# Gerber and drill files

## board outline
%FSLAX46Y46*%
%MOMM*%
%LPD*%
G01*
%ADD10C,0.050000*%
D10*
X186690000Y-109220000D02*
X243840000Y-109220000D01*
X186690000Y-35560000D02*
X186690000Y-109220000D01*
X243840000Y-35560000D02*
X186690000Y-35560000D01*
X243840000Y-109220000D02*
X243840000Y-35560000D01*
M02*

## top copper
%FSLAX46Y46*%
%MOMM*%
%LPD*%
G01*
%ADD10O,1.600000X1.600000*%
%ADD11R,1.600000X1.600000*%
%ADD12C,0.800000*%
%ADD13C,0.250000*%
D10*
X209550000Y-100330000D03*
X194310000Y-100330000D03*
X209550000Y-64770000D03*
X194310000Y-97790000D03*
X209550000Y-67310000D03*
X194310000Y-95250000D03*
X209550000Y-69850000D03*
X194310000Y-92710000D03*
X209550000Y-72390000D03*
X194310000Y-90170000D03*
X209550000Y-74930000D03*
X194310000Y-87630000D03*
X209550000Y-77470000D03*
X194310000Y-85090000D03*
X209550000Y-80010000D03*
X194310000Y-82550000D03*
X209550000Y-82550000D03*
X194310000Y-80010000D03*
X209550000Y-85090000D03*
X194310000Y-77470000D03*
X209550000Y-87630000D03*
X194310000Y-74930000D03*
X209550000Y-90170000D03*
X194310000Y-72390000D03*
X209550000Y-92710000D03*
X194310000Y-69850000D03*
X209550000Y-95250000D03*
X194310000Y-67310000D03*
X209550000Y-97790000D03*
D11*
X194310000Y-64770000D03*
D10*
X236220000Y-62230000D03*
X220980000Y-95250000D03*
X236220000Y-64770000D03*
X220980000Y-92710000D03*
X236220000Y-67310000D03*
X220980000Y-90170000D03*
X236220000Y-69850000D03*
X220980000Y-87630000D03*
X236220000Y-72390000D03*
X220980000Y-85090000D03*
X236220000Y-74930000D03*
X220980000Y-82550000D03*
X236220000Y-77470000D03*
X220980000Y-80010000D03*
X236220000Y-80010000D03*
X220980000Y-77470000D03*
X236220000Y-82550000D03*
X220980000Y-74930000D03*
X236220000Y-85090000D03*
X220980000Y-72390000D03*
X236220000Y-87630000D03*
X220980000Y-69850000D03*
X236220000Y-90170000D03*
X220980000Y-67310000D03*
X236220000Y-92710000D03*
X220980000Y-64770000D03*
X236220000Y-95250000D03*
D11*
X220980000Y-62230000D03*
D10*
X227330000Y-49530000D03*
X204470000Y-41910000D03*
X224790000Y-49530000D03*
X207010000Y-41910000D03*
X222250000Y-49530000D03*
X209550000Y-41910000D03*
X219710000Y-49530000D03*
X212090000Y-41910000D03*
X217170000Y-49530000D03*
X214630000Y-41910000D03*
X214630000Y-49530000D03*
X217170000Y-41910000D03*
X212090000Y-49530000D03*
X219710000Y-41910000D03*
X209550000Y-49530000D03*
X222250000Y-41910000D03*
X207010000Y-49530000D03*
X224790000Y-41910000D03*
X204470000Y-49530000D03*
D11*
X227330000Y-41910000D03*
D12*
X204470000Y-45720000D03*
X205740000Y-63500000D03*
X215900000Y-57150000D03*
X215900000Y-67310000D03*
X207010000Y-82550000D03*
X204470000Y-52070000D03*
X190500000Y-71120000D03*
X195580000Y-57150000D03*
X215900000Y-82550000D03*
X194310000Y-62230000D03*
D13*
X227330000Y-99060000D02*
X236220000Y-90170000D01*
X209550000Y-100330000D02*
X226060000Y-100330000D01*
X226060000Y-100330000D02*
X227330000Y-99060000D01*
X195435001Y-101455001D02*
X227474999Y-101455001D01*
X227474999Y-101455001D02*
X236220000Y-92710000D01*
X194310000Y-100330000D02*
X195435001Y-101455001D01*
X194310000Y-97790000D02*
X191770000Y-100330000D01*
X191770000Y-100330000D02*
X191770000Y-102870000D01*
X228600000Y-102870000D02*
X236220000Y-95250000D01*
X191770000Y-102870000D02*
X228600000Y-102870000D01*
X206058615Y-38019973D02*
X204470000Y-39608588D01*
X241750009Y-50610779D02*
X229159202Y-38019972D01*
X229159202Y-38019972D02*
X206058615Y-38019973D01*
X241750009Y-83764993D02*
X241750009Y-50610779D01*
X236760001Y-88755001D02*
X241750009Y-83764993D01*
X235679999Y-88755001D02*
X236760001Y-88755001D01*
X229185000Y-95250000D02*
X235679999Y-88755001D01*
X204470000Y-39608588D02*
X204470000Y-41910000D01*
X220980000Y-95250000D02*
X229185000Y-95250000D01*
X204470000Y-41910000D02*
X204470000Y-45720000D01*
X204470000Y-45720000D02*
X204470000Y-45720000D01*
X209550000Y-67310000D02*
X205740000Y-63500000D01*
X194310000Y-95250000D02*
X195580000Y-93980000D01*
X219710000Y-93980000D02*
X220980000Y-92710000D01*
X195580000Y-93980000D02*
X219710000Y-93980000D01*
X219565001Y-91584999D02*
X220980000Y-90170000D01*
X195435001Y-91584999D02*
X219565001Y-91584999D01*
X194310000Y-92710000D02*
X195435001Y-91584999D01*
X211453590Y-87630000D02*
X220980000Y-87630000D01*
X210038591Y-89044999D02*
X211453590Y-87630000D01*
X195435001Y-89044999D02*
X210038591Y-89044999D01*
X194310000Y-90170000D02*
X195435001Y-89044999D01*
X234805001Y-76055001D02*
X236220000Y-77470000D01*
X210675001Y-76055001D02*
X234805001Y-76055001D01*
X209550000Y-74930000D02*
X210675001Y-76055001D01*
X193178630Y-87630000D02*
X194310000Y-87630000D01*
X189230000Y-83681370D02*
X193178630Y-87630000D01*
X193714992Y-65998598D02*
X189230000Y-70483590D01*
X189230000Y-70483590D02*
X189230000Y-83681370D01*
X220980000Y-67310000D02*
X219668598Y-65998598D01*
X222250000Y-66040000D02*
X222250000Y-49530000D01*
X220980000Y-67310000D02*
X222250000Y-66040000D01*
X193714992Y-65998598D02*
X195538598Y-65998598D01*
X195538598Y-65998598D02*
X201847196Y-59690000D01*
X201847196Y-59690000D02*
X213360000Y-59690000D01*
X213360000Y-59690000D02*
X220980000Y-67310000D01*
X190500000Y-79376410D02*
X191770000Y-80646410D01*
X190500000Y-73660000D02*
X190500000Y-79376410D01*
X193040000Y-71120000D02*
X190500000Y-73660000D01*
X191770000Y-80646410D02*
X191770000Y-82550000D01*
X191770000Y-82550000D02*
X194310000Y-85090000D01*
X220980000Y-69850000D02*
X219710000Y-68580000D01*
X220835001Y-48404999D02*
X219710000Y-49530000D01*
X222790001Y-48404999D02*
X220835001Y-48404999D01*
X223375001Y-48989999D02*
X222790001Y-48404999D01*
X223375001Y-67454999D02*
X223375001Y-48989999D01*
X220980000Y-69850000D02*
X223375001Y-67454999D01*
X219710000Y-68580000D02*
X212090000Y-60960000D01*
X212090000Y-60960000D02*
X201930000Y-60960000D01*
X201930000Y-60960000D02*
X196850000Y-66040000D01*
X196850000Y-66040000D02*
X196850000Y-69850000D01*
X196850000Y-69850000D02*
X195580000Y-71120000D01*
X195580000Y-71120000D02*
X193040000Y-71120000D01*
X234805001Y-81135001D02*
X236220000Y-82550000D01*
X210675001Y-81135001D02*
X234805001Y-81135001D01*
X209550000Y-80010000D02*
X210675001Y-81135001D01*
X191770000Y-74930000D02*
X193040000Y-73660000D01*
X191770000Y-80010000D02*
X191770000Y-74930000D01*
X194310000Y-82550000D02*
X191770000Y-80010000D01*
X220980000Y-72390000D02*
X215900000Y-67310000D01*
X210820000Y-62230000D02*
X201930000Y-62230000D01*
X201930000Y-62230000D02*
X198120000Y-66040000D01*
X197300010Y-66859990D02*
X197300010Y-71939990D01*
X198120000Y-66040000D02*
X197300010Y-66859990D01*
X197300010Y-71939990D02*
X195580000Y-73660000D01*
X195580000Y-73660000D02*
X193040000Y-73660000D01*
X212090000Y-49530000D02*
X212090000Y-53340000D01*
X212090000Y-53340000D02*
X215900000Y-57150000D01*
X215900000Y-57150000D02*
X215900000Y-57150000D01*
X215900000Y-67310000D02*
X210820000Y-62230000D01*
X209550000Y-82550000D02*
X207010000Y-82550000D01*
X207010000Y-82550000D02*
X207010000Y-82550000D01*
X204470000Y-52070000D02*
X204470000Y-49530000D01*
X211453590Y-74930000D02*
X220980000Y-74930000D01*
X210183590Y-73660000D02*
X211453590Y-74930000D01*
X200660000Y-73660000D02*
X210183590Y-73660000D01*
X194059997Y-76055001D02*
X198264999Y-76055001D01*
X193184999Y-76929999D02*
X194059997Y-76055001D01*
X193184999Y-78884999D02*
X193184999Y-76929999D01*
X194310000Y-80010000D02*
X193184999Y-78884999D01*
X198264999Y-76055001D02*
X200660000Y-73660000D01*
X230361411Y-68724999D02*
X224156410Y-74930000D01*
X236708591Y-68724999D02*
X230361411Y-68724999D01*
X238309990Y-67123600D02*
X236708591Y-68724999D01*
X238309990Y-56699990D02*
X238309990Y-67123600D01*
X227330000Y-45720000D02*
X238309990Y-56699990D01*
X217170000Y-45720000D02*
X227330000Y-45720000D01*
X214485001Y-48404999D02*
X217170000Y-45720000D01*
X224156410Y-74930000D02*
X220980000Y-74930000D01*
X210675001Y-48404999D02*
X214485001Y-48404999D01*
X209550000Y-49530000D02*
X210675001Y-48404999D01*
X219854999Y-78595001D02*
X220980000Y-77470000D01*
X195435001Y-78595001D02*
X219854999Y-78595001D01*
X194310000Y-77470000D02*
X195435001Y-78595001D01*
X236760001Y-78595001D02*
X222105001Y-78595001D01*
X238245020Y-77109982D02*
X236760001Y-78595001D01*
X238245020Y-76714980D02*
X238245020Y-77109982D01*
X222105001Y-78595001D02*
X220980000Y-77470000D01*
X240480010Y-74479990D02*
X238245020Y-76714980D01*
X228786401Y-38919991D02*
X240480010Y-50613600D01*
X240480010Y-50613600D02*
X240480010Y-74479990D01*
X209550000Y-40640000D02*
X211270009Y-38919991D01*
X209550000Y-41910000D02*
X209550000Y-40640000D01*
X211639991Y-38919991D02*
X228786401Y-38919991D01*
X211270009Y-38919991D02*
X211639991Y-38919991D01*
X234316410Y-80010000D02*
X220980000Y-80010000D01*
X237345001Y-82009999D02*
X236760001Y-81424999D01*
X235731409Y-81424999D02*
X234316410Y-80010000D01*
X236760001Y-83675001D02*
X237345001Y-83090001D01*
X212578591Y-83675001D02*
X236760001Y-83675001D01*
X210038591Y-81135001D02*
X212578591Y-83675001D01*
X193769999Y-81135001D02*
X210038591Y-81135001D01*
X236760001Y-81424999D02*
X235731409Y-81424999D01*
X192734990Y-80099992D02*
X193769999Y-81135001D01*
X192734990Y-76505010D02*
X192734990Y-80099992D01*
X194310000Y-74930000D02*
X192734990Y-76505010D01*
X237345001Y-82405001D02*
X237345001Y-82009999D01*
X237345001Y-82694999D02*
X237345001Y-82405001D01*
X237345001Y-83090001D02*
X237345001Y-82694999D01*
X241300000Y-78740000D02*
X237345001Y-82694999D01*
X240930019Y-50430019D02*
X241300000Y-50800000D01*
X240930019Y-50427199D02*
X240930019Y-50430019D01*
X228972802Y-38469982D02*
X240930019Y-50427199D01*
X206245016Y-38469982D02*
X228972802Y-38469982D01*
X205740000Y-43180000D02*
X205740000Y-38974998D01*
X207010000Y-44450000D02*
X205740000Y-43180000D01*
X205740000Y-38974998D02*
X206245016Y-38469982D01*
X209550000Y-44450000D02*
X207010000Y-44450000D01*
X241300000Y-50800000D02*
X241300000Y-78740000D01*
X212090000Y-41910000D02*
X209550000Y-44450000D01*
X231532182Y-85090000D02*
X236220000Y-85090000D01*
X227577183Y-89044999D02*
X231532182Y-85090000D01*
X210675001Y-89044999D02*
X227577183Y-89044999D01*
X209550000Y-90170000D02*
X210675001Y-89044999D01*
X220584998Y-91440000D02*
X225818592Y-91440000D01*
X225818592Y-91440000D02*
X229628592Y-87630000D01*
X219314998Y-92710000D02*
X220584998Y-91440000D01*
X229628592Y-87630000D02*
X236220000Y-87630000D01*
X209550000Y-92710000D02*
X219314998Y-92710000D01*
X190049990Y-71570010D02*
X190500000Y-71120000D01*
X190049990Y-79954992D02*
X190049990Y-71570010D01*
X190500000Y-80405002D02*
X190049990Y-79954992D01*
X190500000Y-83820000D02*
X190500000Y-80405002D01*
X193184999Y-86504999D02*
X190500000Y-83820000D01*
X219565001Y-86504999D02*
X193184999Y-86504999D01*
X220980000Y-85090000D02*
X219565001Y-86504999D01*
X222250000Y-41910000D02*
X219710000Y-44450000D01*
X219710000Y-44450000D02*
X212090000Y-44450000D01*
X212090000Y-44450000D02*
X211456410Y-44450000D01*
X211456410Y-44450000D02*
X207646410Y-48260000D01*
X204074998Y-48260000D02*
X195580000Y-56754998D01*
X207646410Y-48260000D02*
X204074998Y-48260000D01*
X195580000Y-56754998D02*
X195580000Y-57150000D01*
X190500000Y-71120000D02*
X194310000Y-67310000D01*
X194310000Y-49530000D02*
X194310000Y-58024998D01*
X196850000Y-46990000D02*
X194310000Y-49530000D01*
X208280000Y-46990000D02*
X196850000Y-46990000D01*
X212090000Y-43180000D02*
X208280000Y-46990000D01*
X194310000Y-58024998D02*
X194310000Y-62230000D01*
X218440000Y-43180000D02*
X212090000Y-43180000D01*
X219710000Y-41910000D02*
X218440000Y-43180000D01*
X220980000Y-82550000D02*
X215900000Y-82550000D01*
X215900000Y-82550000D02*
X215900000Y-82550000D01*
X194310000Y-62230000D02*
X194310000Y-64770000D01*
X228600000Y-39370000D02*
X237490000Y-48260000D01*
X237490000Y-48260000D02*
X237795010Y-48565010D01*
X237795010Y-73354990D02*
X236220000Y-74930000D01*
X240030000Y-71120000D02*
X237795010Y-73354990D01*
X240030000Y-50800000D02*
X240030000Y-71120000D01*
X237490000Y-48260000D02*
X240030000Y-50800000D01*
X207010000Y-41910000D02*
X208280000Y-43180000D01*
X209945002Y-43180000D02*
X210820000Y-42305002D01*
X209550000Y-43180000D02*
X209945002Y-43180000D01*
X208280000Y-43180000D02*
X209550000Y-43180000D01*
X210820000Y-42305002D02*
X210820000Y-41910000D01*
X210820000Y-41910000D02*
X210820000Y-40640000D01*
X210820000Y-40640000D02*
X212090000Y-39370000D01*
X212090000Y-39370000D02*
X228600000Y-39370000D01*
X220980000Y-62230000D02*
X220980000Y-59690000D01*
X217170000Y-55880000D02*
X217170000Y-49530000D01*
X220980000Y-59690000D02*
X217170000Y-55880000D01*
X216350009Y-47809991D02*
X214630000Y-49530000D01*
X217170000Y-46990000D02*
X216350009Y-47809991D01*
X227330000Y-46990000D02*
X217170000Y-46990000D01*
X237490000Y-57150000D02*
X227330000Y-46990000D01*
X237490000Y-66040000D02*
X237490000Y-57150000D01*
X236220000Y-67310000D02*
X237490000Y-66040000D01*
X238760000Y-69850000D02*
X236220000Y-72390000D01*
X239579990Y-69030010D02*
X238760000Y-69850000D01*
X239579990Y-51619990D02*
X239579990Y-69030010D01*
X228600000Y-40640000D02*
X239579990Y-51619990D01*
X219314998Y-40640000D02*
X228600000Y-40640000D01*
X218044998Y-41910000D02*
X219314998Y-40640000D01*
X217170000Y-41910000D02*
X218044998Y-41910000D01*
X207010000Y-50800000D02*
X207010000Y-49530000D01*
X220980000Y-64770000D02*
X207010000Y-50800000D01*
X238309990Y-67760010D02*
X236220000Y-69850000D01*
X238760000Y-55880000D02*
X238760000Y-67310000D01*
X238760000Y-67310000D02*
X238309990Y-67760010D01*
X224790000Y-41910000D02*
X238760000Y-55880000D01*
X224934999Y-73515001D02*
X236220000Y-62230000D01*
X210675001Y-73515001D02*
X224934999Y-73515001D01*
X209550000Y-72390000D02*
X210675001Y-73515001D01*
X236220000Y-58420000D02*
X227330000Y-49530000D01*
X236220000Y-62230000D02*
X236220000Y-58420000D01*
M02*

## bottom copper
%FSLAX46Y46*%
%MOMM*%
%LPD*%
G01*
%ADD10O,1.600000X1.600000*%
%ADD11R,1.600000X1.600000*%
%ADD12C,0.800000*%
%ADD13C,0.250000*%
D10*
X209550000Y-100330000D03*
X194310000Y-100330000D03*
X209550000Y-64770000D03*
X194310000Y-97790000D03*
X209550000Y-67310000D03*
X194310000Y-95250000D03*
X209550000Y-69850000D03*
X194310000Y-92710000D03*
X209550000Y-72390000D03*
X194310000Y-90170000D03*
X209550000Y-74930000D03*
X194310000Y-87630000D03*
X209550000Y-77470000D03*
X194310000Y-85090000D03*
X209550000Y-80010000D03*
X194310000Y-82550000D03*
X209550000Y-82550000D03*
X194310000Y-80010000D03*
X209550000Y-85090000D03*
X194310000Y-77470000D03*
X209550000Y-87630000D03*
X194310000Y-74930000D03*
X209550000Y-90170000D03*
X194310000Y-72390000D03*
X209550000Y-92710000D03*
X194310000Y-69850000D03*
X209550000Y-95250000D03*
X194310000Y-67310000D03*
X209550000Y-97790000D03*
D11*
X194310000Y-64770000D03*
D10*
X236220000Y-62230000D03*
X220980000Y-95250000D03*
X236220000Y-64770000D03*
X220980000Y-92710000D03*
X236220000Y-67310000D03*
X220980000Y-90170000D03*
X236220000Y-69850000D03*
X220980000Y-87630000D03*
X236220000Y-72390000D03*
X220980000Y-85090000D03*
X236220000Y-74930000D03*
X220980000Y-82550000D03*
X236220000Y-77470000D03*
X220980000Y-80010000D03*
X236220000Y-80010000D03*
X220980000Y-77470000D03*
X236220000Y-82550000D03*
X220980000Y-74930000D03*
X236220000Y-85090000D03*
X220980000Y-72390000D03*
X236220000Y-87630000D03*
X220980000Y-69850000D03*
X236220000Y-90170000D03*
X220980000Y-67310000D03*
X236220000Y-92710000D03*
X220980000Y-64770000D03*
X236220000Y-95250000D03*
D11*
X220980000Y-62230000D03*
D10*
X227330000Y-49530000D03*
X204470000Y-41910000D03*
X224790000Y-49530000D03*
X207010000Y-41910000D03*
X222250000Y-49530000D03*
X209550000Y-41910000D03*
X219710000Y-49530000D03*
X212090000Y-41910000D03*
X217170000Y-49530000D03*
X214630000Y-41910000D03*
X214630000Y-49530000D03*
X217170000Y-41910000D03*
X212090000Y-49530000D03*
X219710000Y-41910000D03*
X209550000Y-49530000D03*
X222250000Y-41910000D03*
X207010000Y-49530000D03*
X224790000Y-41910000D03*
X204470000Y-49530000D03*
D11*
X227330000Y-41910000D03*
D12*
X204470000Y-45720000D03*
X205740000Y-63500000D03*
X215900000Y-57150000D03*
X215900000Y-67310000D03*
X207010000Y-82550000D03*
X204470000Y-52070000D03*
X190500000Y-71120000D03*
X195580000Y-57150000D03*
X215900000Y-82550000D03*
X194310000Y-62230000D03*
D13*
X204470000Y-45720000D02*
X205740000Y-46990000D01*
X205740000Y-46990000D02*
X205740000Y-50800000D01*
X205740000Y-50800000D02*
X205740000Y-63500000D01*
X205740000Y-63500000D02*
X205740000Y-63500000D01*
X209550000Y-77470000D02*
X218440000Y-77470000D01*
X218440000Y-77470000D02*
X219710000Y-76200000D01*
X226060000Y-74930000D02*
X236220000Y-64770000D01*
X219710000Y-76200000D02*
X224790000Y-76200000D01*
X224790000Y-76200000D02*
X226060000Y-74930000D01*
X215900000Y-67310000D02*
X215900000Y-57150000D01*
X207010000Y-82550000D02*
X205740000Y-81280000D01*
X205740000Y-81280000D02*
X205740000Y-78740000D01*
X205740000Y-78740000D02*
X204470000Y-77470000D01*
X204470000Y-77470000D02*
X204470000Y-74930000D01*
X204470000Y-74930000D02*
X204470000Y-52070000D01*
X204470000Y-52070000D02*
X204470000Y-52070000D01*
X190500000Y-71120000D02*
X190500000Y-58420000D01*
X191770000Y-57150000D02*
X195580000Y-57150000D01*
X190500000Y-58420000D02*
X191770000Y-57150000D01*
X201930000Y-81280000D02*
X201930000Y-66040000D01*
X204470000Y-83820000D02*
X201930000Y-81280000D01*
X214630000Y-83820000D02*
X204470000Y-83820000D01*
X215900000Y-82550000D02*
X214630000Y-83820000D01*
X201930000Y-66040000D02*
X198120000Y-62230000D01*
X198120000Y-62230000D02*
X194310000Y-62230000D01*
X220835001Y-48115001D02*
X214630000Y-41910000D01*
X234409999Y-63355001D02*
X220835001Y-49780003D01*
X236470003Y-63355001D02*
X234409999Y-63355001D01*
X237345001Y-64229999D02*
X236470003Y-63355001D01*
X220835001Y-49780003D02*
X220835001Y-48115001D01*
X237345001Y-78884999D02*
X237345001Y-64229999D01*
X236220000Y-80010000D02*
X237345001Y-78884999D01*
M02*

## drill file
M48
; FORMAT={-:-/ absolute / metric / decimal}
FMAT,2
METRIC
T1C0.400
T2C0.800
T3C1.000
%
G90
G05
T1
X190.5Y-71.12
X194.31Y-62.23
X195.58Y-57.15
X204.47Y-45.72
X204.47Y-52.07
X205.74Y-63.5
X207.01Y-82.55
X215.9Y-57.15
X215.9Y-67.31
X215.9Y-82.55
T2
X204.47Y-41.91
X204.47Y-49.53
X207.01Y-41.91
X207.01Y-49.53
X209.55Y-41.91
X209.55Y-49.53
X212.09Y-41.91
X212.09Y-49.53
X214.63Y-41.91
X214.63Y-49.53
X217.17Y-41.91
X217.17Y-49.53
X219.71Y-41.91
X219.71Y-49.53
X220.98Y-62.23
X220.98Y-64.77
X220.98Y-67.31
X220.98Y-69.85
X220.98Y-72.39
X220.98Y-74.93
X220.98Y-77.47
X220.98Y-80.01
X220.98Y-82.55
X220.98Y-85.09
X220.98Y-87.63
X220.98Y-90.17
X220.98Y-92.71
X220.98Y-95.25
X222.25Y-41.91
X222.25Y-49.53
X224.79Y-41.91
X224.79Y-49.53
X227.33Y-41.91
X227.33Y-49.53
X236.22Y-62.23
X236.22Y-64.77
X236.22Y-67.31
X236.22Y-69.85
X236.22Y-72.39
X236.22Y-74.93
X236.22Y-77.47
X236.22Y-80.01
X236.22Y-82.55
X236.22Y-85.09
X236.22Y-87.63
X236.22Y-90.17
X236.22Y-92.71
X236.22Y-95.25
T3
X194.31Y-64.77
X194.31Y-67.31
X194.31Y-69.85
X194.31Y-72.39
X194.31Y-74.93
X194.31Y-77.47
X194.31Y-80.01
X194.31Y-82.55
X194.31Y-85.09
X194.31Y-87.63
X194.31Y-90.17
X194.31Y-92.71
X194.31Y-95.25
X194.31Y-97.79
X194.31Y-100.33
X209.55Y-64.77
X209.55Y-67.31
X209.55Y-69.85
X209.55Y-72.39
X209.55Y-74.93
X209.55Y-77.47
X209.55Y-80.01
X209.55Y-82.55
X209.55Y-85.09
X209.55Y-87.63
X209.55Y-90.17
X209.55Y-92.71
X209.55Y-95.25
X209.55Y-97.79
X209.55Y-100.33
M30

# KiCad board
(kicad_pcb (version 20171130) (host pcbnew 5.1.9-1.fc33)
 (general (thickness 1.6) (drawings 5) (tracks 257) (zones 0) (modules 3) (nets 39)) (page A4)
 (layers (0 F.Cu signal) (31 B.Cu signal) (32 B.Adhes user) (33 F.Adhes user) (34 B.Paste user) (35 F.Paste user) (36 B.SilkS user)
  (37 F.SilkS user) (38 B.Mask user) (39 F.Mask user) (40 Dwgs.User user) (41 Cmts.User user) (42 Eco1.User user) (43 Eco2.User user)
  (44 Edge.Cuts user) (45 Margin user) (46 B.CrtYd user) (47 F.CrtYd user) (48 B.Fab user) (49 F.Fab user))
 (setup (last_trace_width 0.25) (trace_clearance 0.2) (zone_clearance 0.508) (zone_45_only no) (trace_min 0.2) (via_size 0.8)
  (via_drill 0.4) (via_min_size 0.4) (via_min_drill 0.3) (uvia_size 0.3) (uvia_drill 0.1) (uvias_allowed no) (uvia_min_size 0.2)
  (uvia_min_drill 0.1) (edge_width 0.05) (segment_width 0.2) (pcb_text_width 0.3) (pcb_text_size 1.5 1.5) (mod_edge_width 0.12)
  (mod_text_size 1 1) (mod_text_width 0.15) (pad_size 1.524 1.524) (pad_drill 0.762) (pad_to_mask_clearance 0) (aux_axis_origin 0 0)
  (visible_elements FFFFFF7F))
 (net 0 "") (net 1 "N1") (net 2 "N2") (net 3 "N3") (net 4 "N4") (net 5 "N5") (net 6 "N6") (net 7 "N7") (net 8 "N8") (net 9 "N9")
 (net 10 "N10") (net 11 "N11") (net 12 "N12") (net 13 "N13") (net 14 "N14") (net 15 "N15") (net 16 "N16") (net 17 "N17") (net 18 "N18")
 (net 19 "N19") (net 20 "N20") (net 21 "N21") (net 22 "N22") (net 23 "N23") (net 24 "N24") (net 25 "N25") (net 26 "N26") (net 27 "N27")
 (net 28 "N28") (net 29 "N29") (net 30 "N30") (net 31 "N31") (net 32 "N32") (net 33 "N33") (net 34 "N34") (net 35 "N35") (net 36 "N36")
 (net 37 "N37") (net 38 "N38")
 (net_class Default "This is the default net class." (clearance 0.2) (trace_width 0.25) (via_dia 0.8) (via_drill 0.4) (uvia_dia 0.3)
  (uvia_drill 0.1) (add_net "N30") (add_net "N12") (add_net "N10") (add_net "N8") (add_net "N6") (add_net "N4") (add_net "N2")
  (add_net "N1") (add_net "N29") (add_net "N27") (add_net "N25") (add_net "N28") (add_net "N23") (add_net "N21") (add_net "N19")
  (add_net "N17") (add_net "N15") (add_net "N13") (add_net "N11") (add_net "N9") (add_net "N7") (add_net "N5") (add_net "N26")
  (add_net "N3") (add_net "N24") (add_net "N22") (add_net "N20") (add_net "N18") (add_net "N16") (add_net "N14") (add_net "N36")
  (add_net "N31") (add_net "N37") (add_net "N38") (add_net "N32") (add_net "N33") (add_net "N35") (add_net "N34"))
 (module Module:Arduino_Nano (layer F.Cu) (at 194.31 64.77)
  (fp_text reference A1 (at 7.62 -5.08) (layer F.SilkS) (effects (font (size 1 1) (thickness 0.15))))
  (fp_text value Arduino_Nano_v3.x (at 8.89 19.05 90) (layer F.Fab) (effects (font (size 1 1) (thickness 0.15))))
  (pad 16 thru_hole oval (at 15.24 35.56) (size 1.6 1.6) (drill 1) (layers *.Cu *.Mask) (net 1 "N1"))
  (pad 15 thru_hole oval (at 0 35.56) (size 1.6 1.6) (drill 1) (layers *.Cu *.Mask) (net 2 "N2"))
  (pad 30 thru_hole oval (at 15.24 0) (size 1.6 1.6) (drill 1) (layers *.Cu *.Mask) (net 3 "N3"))
  (pad 14 thru_hole oval (at 0 33.02) (size 1.6 1.6) (drill 1) (layers *.Cu *.Mask) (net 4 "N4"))
  (pad 29 thru_hole oval (at 15.24 2.54) (size 1.6 1.6) (drill 1) (layers *.Cu *.Mask) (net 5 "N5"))
  (pad 13 thru_hole oval (at 0 30.48) (size 1.6 1.6) (drill 1) (layers *.Cu *.Mask) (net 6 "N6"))
  (pad 28 thru_hole oval (at 15.24 5.08) (size 1.6 1.6) (drill 1) (layers *.Cu *.Mask) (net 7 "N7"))
  (pad 12 thru_hole oval (at 0 27.94) (size 1.6 1.6) (drill 1) (layers *.Cu *.Mask) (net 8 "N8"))
  (pad 27 thru_hole oval (at 15.24 7.62) (size 1.6 1.6) (drill 1) (layers *.Cu *.Mask) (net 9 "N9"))
  (pad 11 thru_hole oval (at 0 25.4) (size 1.6 1.6) (drill 1) (layers *.Cu *.Mask) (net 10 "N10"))
  (pad 26 thru_hole oval (at 15.24 10.16) (size 1.6 1.6) (drill 1) (layers *.Cu *.Mask) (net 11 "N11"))
  (pad 10 thru_hole oval (at 0 22.86) (size 1.6 1.6) (drill 1) (layers *.Cu *.Mask) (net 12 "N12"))
  (pad 25 thru_hole oval (at 15.24 12.7) (size 1.6 1.6) (drill 1) (layers *.Cu *.Mask) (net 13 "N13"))
  (pad 9 thru_hole oval (at 0 20.32) (size 1.6 1.6) (drill 1) (layers *.Cu *.Mask) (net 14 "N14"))
  (pad 24 thru_hole oval (at 15.24 15.24) (size 1.6 1.6) (drill 1) (layers *.Cu *.Mask) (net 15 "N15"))
  (pad 8 thru_hole oval (at 0 17.78) (size 1.6 1.6) (drill 1) (layers *.Cu *.Mask) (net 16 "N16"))
  (pad 23 thru_hole oval (at 15.24 17.78) (size 1.6 1.6) (drill 1) (layers *.Cu *.Mask) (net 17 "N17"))
  (pad 7 thru_hole oval (at 0 15.24) (size 1.6 1.6) (drill 1) (layers *.Cu *.Mask) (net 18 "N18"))
  (pad 22 thru_hole oval (at 15.24 20.32) (size 1.6 1.6) (drill 1) (layers *.Cu *.Mask) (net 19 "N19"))
  (pad 6 thru_hole oval (at 0 12.7) (size 1.6 1.6) (drill 1) (layers *.Cu *.Mask) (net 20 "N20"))
  (pad 21 thru_hole oval (at 15.24 22.86) (size 1.6 1.6) (drill 1) (layers *.Cu *.Mask) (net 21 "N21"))
  (pad 5 thru_hole oval (at 0 10.16) (size 1.6 1.6) (drill 1) (layers *.Cu *.Mask) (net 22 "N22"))
  (pad 20 thru_hole oval (at 15.24 25.4) (size 1.6 1.6) (drill 1) (layers *.Cu *.Mask) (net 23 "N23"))
  (pad 4 thru_hole oval (at 0 7.62) (size 1.6 1.6) (drill 1) (layers *.Cu *.Mask) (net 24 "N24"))
  (pad 19 thru_hole oval (at 15.24 27.94) (size 1.6 1.6) (drill 1) (layers *.Cu *.Mask) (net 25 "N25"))
  (pad 3 thru_hole oval (at 0 5.08) (size 1.6 1.6) (drill 1) (layers *.Cu *.Mask) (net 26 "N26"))
  (pad 18 thru_hole oval (at 15.24 30.48) (size 1.6 1.6) (drill 1) (layers *.Cu *.Mask) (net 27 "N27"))
  (pad 2 thru_hole oval (at 0 2.54) (size 1.6 1.6) (drill 1) (layers *.Cu *.Mask) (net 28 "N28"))
  (pad 17 thru_hole oval (at 15.24 33.02) (size 1.6 1.6) (drill 1) (layers *.Cu *.Mask) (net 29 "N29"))
  (pad 1 thru_hole rect (at 0 0) (size 1.6 1.6) (drill 1) (layers *.Cu *.Mask) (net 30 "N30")))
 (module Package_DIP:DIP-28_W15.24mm (layer F.Cu) (at 220.98 62.23)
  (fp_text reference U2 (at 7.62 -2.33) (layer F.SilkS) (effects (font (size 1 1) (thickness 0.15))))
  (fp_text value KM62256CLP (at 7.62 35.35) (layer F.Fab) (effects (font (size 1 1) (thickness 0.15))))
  (pad 28 thru_hole oval (at 15.24 0) (size 1.6 1.6) (drill 0.8) (layers *.Cu *.Mask) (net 9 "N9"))
  (pad 14 thru_hole oval (at 0 33.02) (size 1.6 1.6) (drill 0.8) (layers *.Cu *.Mask) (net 5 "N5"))
  (pad 27 thru_hole oval (at 15.24 2.54) (size 1.6 1.6) (drill 0.8) (layers *.Cu *.Mask) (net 13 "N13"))
  (pad 13 thru_hole oval (at 0 30.48) (size 1.6 1.6) (drill 0.8) (layers *.Cu *.Mask) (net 6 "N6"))
  (pad 26 thru_hole oval (at 15.24 5.08) (size 1.6 1.6) (drill 0.8) (layers *.Cu *.Mask) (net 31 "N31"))
  (pad 12 thru_hole oval (at 0 27.94) (size 1.6 1.6) (drill 0.8) (layers *.Cu *.Mask) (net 8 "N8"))
  (pad 25 thru_hole oval (at 15.24 7.62) (size 1.6 1.6) (drill 0.8) (layers *.Cu *.Mask) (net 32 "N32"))
  (pad 11 thru_hole oval (at 0 25.4) (size 1.6 1.6) (drill 0.8) (layers *.Cu *.Mask) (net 10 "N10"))
  (pad 24 thru_hole oval (at 15.24 10.16) (size 1.6 1.6) (drill 0.8) (layers *.Cu *.Mask) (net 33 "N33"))
  (pad 10 thru_hole oval (at 0 22.86) (size 1.6 1.6) (drill 0.8) (layers *.Cu *.Mask) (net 28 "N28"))
  (pad 23 thru_hole oval (at 15.24 12.7) (size 1.6 1.6) (drill 0.8) (layers *.Cu *.Mask) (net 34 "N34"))
  (pad 9 thru_hole oval (at 0 20.32) (size 1.6 1.6) (drill 0.8) (layers *.Cu *.Mask) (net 30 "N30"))
  (pad 22 thru_hole oval (at 15.24 15.24) (size 1.6 1.6) (drill 0.8) (layers *.Cu *.Mask) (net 11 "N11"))
  (pad 8 thru_hole oval (at 0 17.78) (size 1.6 1.6) (drill 0.8) (layers *.Cu *.Mask) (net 22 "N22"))
  (pad 21 thru_hole oval (at 15.24 17.78) (size 1.6 1.6) (drill 0.8) (layers *.Cu *.Mask) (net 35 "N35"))
  (pad 7 thru_hole oval (at 0 15.24) (size 1.6 1.6) (drill 0.8) (layers *.Cu *.Mask) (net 20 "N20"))
  (pad 20 thru_hole oval (at 15.24 20.32) (size 1.6 1.6) (drill 0.8) (layers *.Cu *.Mask) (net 15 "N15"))
  (pad 6 thru_hole oval (at 0 12.7) (size 1.6 1.6) (drill 0.8) (layers *.Cu *.Mask) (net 18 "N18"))
  (pad 19 thru_hole oval (at 15.24 22.86) (size 1.6 1.6) (drill 0.8) (layers *.Cu *.Mask) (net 23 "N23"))
  (pad 5 thru_hole oval (at 0 10.16) (size 1.6 1.6) (drill 0.8) (layers *.Cu *.Mask) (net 16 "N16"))
  (pad 18 thru_hole oval (at 15.24 25.4) (size 1.6 1.6) (drill 0.8) (layers *.Cu *.Mask) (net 25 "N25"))
  (pad 4 thru_hole oval (at 0 7.62) (size 1.6 1.6) (drill 0.8) (layers *.Cu *.Mask) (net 14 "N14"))
  (pad 17 thru_hole oval (at 15.24 27.94) (size 1.6 1.6) (drill 0.8) (layers *.Cu *.Mask) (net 1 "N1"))
  (pad 3 thru_hole oval (at 0 5.08) (size 1.6 1.6) (drill 0.8) (layers *.Cu *.Mask) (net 12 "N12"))
  (pad 16 thru_hole oval (at 15.24 30.48) (size 1.6 1.6) (drill 0.8) (layers *.Cu *.Mask) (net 2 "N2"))
  (pad 2 thru_hole oval (at 0 2.54) (size 1.6 1.6) (drill 0.8) (layers *.Cu *.Mask) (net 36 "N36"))
  (pad 15 thru_hole oval (at 15.24 33.02) (size 1.6 1.6) (drill 0.8) (layers *.Cu *.Mask) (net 4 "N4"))
  (pad 1 thru_hole rect (at 0 0) (size 1.6 1.6) (drill 0.8) (layers *.Cu *.Mask) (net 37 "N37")))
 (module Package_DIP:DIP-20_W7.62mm (layer F.Cu) (at 227.33 41.91 270)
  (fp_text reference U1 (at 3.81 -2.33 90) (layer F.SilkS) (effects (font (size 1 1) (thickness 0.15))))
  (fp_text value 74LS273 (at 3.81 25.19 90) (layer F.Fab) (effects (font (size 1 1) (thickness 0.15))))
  (pad 20 thru_hole oval (at 7.62 0 270) (size 1.6 1.6) (drill 0.8) (layers *.Cu *.Mask) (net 9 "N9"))
  (pad 10 thru_hole oval (at 0 22.86 270) (size 1.6 1.6) (drill 0.8) (layers *.Cu *.Mask) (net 5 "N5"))
  (pad 19 thru_hole oval (at 7.62 2.54 270) (size 1.6 1.6) (drill 0.8) (layers *.Cu *.Mask) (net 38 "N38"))
  (pad 9 thru_hole oval (at 0 20.32 270) (size 1.6 1.6) (drill 0.8) (layers *.Cu *.Mask) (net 34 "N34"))
  (pad 18 thru_hole oval (at 7.62 5.08 270) (size 1.6 1.6) (drill 0.8) (layers *.Cu *.Mask) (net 12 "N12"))
  (pad 8 thru_hole oval (at 0 17.78 270) (size 1.6 1.6) (drill 0.8) (layers *.Cu *.Mask) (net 20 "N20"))
  (pad 17 thru_hole oval (at 7.62 7.62 270) (size 1.6 1.6) (drill 0.8) (layers *.Cu *.Mask) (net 14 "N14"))
  (pad 7 thru_hole oval (at 0 15.24 270) (size 1.6 1.6) (drill 0.8) (layers *.Cu *.Mask) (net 22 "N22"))
  (pad 16 thru_hole oval (at 7.62 10.16 270) (size 1.6 1.6) (drill 0.8) (layers *.Cu *.Mask) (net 37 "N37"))
  (pad 6 thru_hole oval (at 0 12.7 270) (size 1.6 1.6) (drill 0.8) (layers *.Cu *.Mask) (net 35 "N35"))
  (pad 15 thru_hole oval (at 7.62 12.7 270) (size 1.6 1.6) (drill 0.8) (layers *.Cu *.Mask) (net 31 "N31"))
  (pad 5 thru_hole oval (at 0 10.16 270) (size 1.6 1.6) (drill 0.8) (layers *.Cu *.Mask) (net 33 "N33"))
  (pad 14 thru_hole oval (at 7.62 15.24 270) (size 1.6 1.6) (drill 0.8) (layers *.Cu *.Mask) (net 16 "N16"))
  (pad 4 thru_hole oval (at 0 7.62 270) (size 1.6 1.6) (drill 0.8) (layers *.Cu *.Mask) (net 30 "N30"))
  (pad 13 thru_hole oval (at 7.62 17.78 270) (size 1.6 1.6) (drill 0.8) (layers *.Cu *.Mask) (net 18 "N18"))
  (pad 3 thru_hole oval (at 0 5.08 270) (size 1.6 1.6) (drill 0.8) (layers *.Cu *.Mask) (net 28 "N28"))
  (pad 12 thru_hole oval (at 7.62 20.32 270) (size 1.6 1.6) (drill 0.8) (layers *.Cu *.Mask) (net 36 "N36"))
  (pad 2 thru_hole oval (at 0 2.54 270) (size 1.6 1.6) (drill 0.8) (layers *.Cu *.Mask) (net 32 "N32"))
  (pad 11 thru_hole oval (at 7.62 22.86 270) (size 1.6 1.6) (drill 0.8) (layers *.Cu *.Mask) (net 17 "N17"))
  (pad 1 thru_hole rect (at 0 0 270) (size 1.6 1.6) (drill 0.8) (layers *.Cu *.Mask) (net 9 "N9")))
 (gr_line (start 186.69 109.22) (end 243.84 109.22) (layer Edge.Cuts) (width 0.05))
 (gr_line (start 186.69 35.56) (end 186.69 109.22) (layer Edge.Cuts) (width 0.05))
 (gr_line (start 243.84 35.56) (end 186.69 35.56) (layer Edge.Cuts) (width 0.05))
 (gr_line (start 243.84 109.22) (end 243.84 35.56) (layer Edge.Cuts) (width 0.05))
 (segment (start 227.33 99.06) (end 236.22 90.17) (width 0.25) (layer F.Cu) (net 1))
 (segment (start 209.55 100.33) (end 226.06 100.33) (width 0.25) (layer F.Cu) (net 1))
 (segment (start 226.06 100.33) (end 227.33 99.06) (width 0.25) (layer F.Cu) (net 1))
 (segment (start 195.435001 101.455001) (end 227.474999 101.455001) (width 0.25) (layer F.Cu) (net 2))
 (segment (start 227.474999 101.455001) (end 236.22 92.71) (width 0.25) (layer F.Cu) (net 2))
 (segment (start 194.31 100.33) (end 195.435001 101.455001) (width 0.25) (layer F.Cu) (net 2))
 (segment (start 194.31 97.79) (end 191.77 100.33) (width 0.25) (layer F.Cu) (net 4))
 (segment (start 191.77 100.33) (end 191.77 102.87) (width 0.25) (layer F.Cu) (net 4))
 (segment (start 228.6 102.87) (end 236.22 95.25) (width 0.25) (layer F.Cu) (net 4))
 (segment (start 191.77 102.87) (end 228.6 102.87) (width 0.25) (layer F.Cu) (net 4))
 (segment (start 206.058615 38.019973) (end 204.47 39.608588) (width 0.25) (layer F.Cu) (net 5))
 (segment (start 241.750009 50.610779) (end 229.159202 38.019972) (width 0.25) (layer F.Cu) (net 5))
 (segment (start 229.159202 38.019972) (end 206.058615 38.019973) (width 0.25) (layer F.Cu) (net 5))
 (segment (start 241.750009 83.764993) (end 241.750009 50.610779) (width 0.25) (layer F.Cu) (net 5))
 (segment (start 236.760001 88.755001) (end 241.750009 83.764993) (width 0.25) (layer F.Cu) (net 5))
 (segment (start 235.679999 88.755001) (end 236.760001 88.755001) (width 0.25) (layer F.Cu) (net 5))
 (segment (start 229.185 95.25) (end 235.679999 88.755001) (width 0.25) (layer F.Cu) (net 5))
 (segment (start 204.47 39.608588) (end 204.47 41.91) (width 0.25) (layer F.Cu) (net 5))
 (segment (start 220.98 95.25) (end 229.185 95.25) (width 0.25) (layer F.Cu) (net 5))
 (segment (start 204.47 41.91) (end 204.47 45.72) (width 0.25) (layer F.Cu) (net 5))
 (segment (start 204.47 45.72) (end 204.47 45.72) (width 0.25) (layer F.Cu) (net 5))
 (via (at 204.47 45.72) (size 0.8) (drill 0.4) (layers F.Cu B.Cu) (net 5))
 (segment (start 204.47 45.72) (end 205.74 46.99) (width 0.25) (layer B.Cu) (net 5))
 (segment (start 205.74 46.99) (end 205.74 50.8) (width 0.25) (layer B.Cu) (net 5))
 (segment (start 205.74 50.8) (end 205.74 63.5) (width 0.25) (layer B.Cu) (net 5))
 (segment (start 205.74 63.5) (end 205.74 63.5) (width 0.25) (layer B.Cu) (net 5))
 (via (at 205.74 63.5) (size 0.8) (drill 0.4) (layers F.Cu B.Cu) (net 5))
 (segment (start 209.55 67.31) (end 205.74 63.5) (width 0.25) (layer F.Cu) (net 5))
 (segment (start 194.31 95.25) (end 195.58 93.98) (width 0.25) (layer F.Cu) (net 6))
 (segment (start 219.71 93.98) (end 220.98 92.71) (width 0.25) (layer F.Cu) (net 6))
 (segment (start 195.58 93.98) (end 219.71 93.98) (width 0.25) (layer F.Cu) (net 6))
 (segment (start 219.565001 91.584999) (end 220.98 90.17) (width 0.25) (layer F.Cu) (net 8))
 (segment (start 195.435001 91.584999) (end 219.565001 91.584999) (width 0.25) (layer F.Cu) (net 8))
 (segment (start 194.31 92.71) (end 195.435001 91.584999) (width 0.25) (layer F.Cu) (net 8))
 (segment (start 211.45359 87.63) (end 220.98 87.63) (width 0.25) (layer F.Cu) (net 10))
 (segment (start 210.038591 89.044999) (end 211.45359 87.63) (width 0.25) (layer F.Cu) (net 10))
 (segment (start 195.435001 89.044999) (end 210.038591 89.044999) (width 0.25) (layer F.Cu) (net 10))
 (segment (start 194.31 90.17) (end 195.435001 89.044999) (width 0.25) (layer F.Cu) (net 10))
 (segment (start 234.805001 76.055001) (end 236.22 77.47) (width 0.25) (layer F.Cu) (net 11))
 (segment (start 210.675001 76.055001) (end 234.805001 76.055001) (width 0.25) (layer F.Cu) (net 11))
 (segment (start 209.55 74.93) (end 210.675001 76.055001) (width 0.25) (layer F.Cu) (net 11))
 (segment (start 193.17863 87.63) (end 194.31 87.63) (width 0.25) (layer F.Cu) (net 12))
 (segment (start 189.23 83.68137) (end 193.17863 87.63) (width 0.25) (layer F.Cu) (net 12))
 (segment (start 193.714992 65.998598) (end 189.23 70.48359) (width 0.25) (layer F.Cu) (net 12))
 (segment (start 189.23 70.48359) (end 189.23 83.68137) (width 0.25) (layer F.Cu) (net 12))
 (segment (start 220.98 67.31) (end 219.668598 65.998598) (width 0.25) (layer F.Cu) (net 12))
 (segment (start 222.25 66.04) (end 222.25 49.53) (width 0.25) (layer F.Cu) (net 12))
 (segment (start 220.98 67.31) (end 222.25 66.04) (width 0.25) (layer F.Cu) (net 12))
 (segment (start 193.714992 65.998598) (end 195.538598 65.998598) (width 0.25) (layer F.Cu) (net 12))
 (segment (start 195.538598 65.998598) (end 201.847196 59.69) (width 0.25) (layer F.Cu) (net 12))
 (segment (start 201.847196 59.69) (end 213.36 59.69) (width 0.25) (layer F.Cu) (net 12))
 (segment (start 213.36 59.69) (end 220.98 67.31) (width 0.25) (layer F.Cu) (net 12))
 (segment (start 209.55 77.47) (end 218.44 77.47) (width 0.25) (layer B.Cu) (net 13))
 (segment (start 218.44 77.47) (end 219.71 76.2) (width 0.25) (layer B.Cu) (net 13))
 (segment (start 226.06 74.93) (end 236.22 64.77) (width 0.25) (layer B.Cu) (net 13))
 (segment (start 219.71 76.2) (end 224.79 76.2) (width 0.25) (layer B.Cu) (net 13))
 (segment (start 224.79 76.2) (end 226.06 74.93) (width 0.25) (layer B.Cu) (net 13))
 (segment (start 190.5 79.37641) (end 191.77 80.64641) (width 0.25) (layer F.Cu) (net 14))
 (segment (start 190.5 73.66) (end 190.5 79.37641) (width 0.25) (layer F.Cu) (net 14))
 (segment (start 193.04 71.12) (end 190.5 73.66) (width 0.25) (layer F.Cu) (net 14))
 (segment (start 191.77 80.64641) (end 191.77 82.55) (width 0.25) (layer F.Cu) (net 14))
 (segment (start 191.77 82.55) (end 194.31 85.09) (width 0.25) (layer F.Cu) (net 14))
 (segment (start 220.98 69.85) (end 219.71 68.58) (width 0.25) (layer F.Cu) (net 14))
 (segment (start 220.835001 48.404999) (end 219.71 49.53) (width 0.25) (layer F.Cu) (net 14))
 (segment (start 222.790001 48.404999) (end 220.835001 48.404999) (width 0.25) (layer F.Cu) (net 14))
 (segment (start 223.375001 48.989999) (end 222.790001 48.404999) (width 0.25) (layer F.Cu) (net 14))
 (segment (start 223.375001 67.454999) (end 223.375001 48.989999) (width 0.25) (layer F.Cu) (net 14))
 (segment (start 220.98 69.85) (end 223.375001 67.454999) (width 0.25) (layer F.Cu) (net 14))
 (segment (start 219.71 68.58) (end 212.09 60.96) (width 0.25) (layer F.Cu) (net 14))
 (segment (start 212.09 60.96) (end 201.93 60.96) (width 0.25) (layer F.Cu) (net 14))
 (segment (start 201.93 60.96) (end 196.85 66.04) (width 0.25) (layer F.Cu) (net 14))
 (segment (start 196.85 66.04) (end 196.85 69.85) (width 0.25) (layer F.Cu) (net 14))
 (segment (start 196.85 69.85) (end 195.58 71.12) (width 0.25) (layer F.Cu) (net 14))
 (segment (start 195.58 71.12) (end 193.04 71.12) (width 0.25) (layer F.Cu) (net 14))
 (segment (start 234.805001 81.135001) (end 236.22 82.55) (width 0.25) (layer F.Cu) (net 15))
 (segment (start 210.675001 81.135001) (end 234.805001 81.135001) (width 0.25) (layer F.Cu) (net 15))
 (segment (start 209.55 80.01) (end 210.675001 81.135001) (width 0.25) (layer F.Cu) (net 15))
 (segment (start 191.77 74.93) (end 193.04 73.66) (width 0.25) (layer F.Cu) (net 16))
 (segment (start 191.77 80.01) (end 191.77 74.93) (width 0.25) (layer F.Cu) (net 16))
 (segment (start 194.31 82.55) (end 191.77 80.01) (width 0.25) (layer F.Cu) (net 16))
 (segment (start 220.98 72.39) (end 215.9 67.31) (width 0.25) (layer F.Cu) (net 16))
 (segment (start 210.82 62.23) (end 201.93 62.23) (width 0.25) (layer F.Cu) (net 16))
 (segment (start 201.93 62.23) (end 198.12 66.04) (width 0.25) (layer F.Cu) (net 16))
 (segment (start 197.30001 66.85999) (end 197.30001 71.93999) (width 0.25) (layer F.Cu) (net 16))
 (segment (start 198.12 66.04) (end 197.30001 66.85999) (width 0.25) (layer F.Cu) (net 16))
 (segment (start 197.30001 71.93999) (end 195.58 73.66) (width 0.25) (layer F.Cu) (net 16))
 (segment (start 195.58 73.66) (end 193.04 73.66) (width 0.25) (layer F.Cu) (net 16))
 (segment (start 212.09 49.53) (end 212.09 53.34) (width 0.25) (layer F.Cu) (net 16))
 (segment (start 212.09 53.34) (end 215.9 57.15) (width 0.25) (layer F.Cu) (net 16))
 (segment (start 215.9 57.15) (end 215.9 57.15) (width 0.25) (layer F.Cu) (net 16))
 (via (at 215.9 57.15) (size 0.8) (drill 0.4) (layers F.Cu B.Cu) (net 16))
 (segment (start 215.9 67.31) (end 210.82 62.23) (width 0.25) (layer F.Cu) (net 16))
 (via (at 215.9 67.31) (size 0.8) (drill 0.4) (layers F.Cu B.Cu) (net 16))
 (segment (start 215.9 67.31) (end 215.9 57.15) (width 0.25) (layer B.Cu) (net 16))
 (segment (start 209.55 82.55) (end 207.01 82.55) (width 0.25) (layer F.Cu) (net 17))
 (segment (start 207.01 82.55) (end 207.01 82.55) (width 0.25) (layer F.Cu) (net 17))
 (via (at 207.01 82.55) (size 0.8) (drill 0.4) (layers F.Cu B.Cu) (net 17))
 (segment (start 207.01 82.55) (end 205.74 81.28) (width 0.25) (layer B.Cu) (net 17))
 (segment (start 205.74 81.28) (end 205.74 78.74) (width 0.25) (layer B.Cu) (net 17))
 (segment (start 205.74 78.74) (end 204.47 77.47) (width 0.25) (layer B.Cu) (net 17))
 (segment (start 204.47 77.47) (end 204.47 74.93) (width 0.25) (layer B.Cu) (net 17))
 (segment (start 204.47 74.93) (end 204.47 52.07) (width 0.25) (layer B.Cu) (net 17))
 (segment (start 204.47 52.07) (end 204.47 52.07) (width 0.25) (layer B.Cu) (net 17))
 (via (at 204.47 52.07) (size 0.8) (drill 0.4) (layers F.Cu B.Cu) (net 17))
 (segment (start 204.47 52.07) (end 204.47 49.53) (width 0.25) (layer F.Cu) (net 17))
 (segment (start 211.45359 74.93) (end 220.98 74.93) (width 0.25) (layer F.Cu) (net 18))
 (segment (start 210.18359 73.66) (end 211.45359 74.93) (width 0.25) (layer F.Cu) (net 18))
 (segment (start 200.66 73.66) (end 210.18359 73.66) (width 0.25) (layer F.Cu) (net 18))
 (segment (start 194.059997 76.055001) (end 198.264999 76.055001) (width 0.25) (layer F.Cu) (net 18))
 (segment (start 193.184999 76.929999) (end 194.059997 76.055001) (width 0.25) (layer F.Cu) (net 18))
 (segment (start 193.184999 78.884999) (end 193.184999 76.929999) (width 0.25) (layer F.Cu) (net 18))
 (segment (start 194.31 80.01) (end 193.184999 78.884999) (width 0.25) (layer F.Cu) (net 18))
 (segment (start 198.264999 76.055001) (end 200.66 73.66) (width 0.25) (layer F.Cu) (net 18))
 (segment (start 230.361411 68.724999) (end 224.15641 74.93) (width 0.25) (layer F.Cu) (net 18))
 (segment (start 236.708591 68.724999) (end 230.361411 68.724999) (width 0.25) (layer F.Cu) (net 18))
 (segment (start 238.30999 67.1236) (end 236.708591 68.724999) (width 0.25) (layer F.Cu) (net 18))
 (segment (start 238.30999 56.69999) (end 238.30999 67.1236) (width 0.25) (layer F.Cu) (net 18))
 (segment (start 227.33 45.72) (end 238.30999 56.69999) (width 0.25) (layer F.Cu) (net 18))
 (segment (start 217.17 45.72) (end 227.33 45.72) (width 0.25) (layer F.Cu) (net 18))
 (segment (start 214.485001 48.404999) (end 217.17 45.72) (width 0.25) (layer F.Cu) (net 18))
 (segment (start 224.15641 74.93) (end 220.98 74.93) (width 0.25) (layer F.Cu) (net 18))
 (segment (start 210.675001 48.404999) (end 214.485001 48.404999) (width 0.25) (layer F.Cu) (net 18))
 (segment (start 209.55 49.53) (end 210.675001 48.404999) (width 0.25) (layer F.Cu) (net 18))
 (segment (start 219.854999 78.595001) (end 220.98 77.47) (width 0.25) (layer F.Cu) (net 20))
 (segment (start 195.435001 78.595001) (end 219.854999 78.595001) (width 0.25) (layer F.Cu) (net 20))
 (segment (start 194.31 77.47) (end 195.435001 78.595001) (width 0.25) (layer F.Cu) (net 20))
 (segment (start 236.760001 78.595001) (end 222.105001 78.595001) (width 0.25) (layer F.Cu) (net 20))
 (segment (start 238.24502 77.109982) (end 236.760001 78.595001) (width 0.25) (layer F.Cu) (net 20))
 (segment (start 238.24502 76.71498) (end 238.24502 77.109982) (width 0.25) (layer F.Cu) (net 20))
 (segment (start 222.105001 78.595001) (end 220.98 77.47) (width 0.25) (layer F.Cu) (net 20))
 (segment (start 240.48001 74.47999) (end 238.24502 76.71498) (width 0.25) (layer F.Cu) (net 20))
 (segment (start 228.786401 38.919991) (end 240.48001 50.6136) (width 0.25) (layer F.Cu) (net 20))
 (segment (start 240.48001 50.6136) (end 240.48001 74.47999) (width 0.25) (layer F.Cu) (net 20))
 (segment (start 209.55 40.64) (end 211.270009 38.919991) (width 0.25) (layer F.Cu) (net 20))
 (segment (start 209.55 41.91) (end 209.55 40.64) (width 0.25) (layer F.Cu) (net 20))
 (segment (start 211.639991 38.919991) (end 228.786401 38.919991) (width 0.25) (layer F.Cu) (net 20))
 (segment (start 211.270009 38.919991) (end 211.639991 38.919991) (width 0.25) (layer F.Cu) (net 20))
 (segment (start 234.31641 80.01) (end 220.98 80.01) (width 0.25) (layer F.Cu) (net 22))
 (segment (start 237.345001 82.009999) (end 236.760001 81.424999) (width 0.25) (layer F.Cu) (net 22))
 (segment (start 235.731409 81.424999) (end 234.31641 80.01) (width 0.25) (layer F.Cu) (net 22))
 (segment (start 236.760001 83.675001) (end 237.345001 83.090001) (width 0.25) (layer F.Cu) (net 22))
 (segment (start 212.578591 83.675001) (end 236.760001 83.675001) (width 0.25) (layer F.Cu) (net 22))
 (segment (start 210.038591 81.135001) (end 212.578591 83.675001) (width 0.25) (layer F.Cu) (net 22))
 (segment (start 193.769999 81.135001) (end 210.038591 81.135001) (width 0.25) (layer F.Cu) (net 22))
 (segment (start 236.760001 81.424999) (end 235.731409 81.424999) (width 0.25) (layer F.Cu) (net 22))
 (segment (start 192.73499 80.099992) (end 193.769999 81.135001) (width 0.25) (layer F.Cu) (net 22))
 (segment (start 192.73499 76.50501) (end 192.73499 80.099992) (width 0.25) (layer F.Cu) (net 22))
 (segment (start 194.31 74.93) (end 192.73499 76.50501) (width 0.25) (layer F.Cu) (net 22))
 (segment (start 237.345001 82.405001) (end 237.345001 82.009999) (width 0.25) (layer F.Cu) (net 22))
 (segment (start 237.345001 82.694999) (end 237.345001 82.405001) (width 0.25) (layer F.Cu) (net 22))
 (segment (start 237.345001 83.090001) (end 237.345001 82.694999) (width 0.25) (layer F.Cu) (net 22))
 (segment (start 241.3 78.74) (end 237.345001 82.694999) (width 0.25) (layer F.Cu) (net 22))
 (segment (start 240.930019 50.430019) (end 241.3 50.8) (width 0.25) (layer F.Cu) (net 22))
 (segment (start 240.930019 50.427199) (end 240.930019 50.430019) (width 0.25) (layer F.Cu) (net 22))
 (segment (start 228.972802 38.469982) (end 240.930019 50.427199) (width 0.25) (layer F.Cu) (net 22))
 (segment (start 206.245016 38.469982) (end 228.972802 38.469982) (width 0.25) (layer F.Cu) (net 22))
 (segment (start 205.74 43.18) (end 205.74 38.974998) (width 0.25) (layer F.Cu) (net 22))
 (segment (start 207.01 44.45) (end 205.74 43.18) (width 0.25) (layer F.Cu) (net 22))
 (segment (start 205.74 38.974998) (end 206.245016 38.469982) (width 0.25) (layer F.Cu) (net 22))
 (segment (start 209.55 44.45) (end 207.01 44.45) (width 0.25) (layer F.Cu) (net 22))
 (segment (start 241.3 50.8) (end 241.3 78.74) (width 0.25) (layer F.Cu) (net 22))
 (segment (start 212.09 41.91) (end 209.55 44.45) (width 0.25) (layer F.Cu) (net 22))
 (segment (start 231.532182 85.09) (end 236.22 85.09) (width 0.25) (layer F.Cu) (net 23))
 (segment (start 227.577183 89.044999) (end 231.532182 85.09) (width 0.25) (layer F.Cu) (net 23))
 (segment (start 210.675001 89.044999) (end 227.577183 89.044999) (width 0.25) (layer F.Cu) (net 23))
 (segment (start 209.55 90.17) (end 210.675001 89.044999) (width 0.25) (layer F.Cu) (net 23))
 (segment (start 220.584998 91.44) (end 225.818592 91.44) (width 0.25) (layer F.Cu) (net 25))
 (segment (start 225.818592 91.44) (end 229.628592 87.63) (width 0.25) (layer F.Cu) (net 25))
 (segment (start 219.314998 92.71) (end 220.584998 91.44) (width 0.25) (layer F.Cu) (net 25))
 (segment (start 229.628592 87.63) (end 236.22 87.63) (width 0.25) (layer F.Cu) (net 25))
 (segment (start 209.55 92.71) (end 219.314998 92.71) (width 0.25) (layer F.Cu) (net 25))
 (segment (start 190.04999 71.57001) (end 190.5 71.12) (width 0.25) (layer F.Cu) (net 28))
 (segment (start 190.04999 79.954992) (end 190.04999 71.57001) (width 0.25) (layer F.Cu) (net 28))
 (segment (start 190.5 80.405002) (end 190.04999 79.954992) (width 0.25) (layer F.Cu) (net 28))
 (segment (start 190.5 83.82) (end 190.5 80.405002) (width 0.25) (layer F.Cu) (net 28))
 (segment (start 193.184999 86.504999) (end 190.5 83.82) (width 0.25) (layer F.Cu) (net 28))
 (segment (start 219.565001 86.504999) (end 193.184999 86.504999) (width 0.25) (layer F.Cu) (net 28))
 (segment (start 220.98 85.09) (end 219.565001 86.504999) (width 0.25) (layer F.Cu) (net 28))
 (segment (start 222.25 41.91) (end 219.71 44.45) (width 0.25) (layer F.Cu) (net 28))
 (segment (start 219.71 44.45) (end 212.09 44.45) (width 0.25) (layer F.Cu) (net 28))
 (segment (start 212.09 44.45) (end 211.45641 44.45) (width 0.25) (layer F.Cu) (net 28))
 (segment (start 211.45641 44.45) (end 207.64641 48.26) (width 0.25) (layer F.Cu) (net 28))
 (segment (start 204.074998 48.26) (end 195.58 56.754998) (width 0.25) (layer F.Cu) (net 28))
 (segment (start 207.64641 48.26) (end 204.074998 48.26) (width 0.25) (layer F.Cu) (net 28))
 (segment (start 195.58 56.754998) (end 195.58 57.15) (width 0.25) (layer F.Cu) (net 28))
 (segment (start 190.5 71.12) (end 194.31 67.31) (width 0.25) (layer F.Cu) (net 28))
 (via (at 190.5 71.12) (size 0.8) (drill 0.4) (layers F.Cu B.Cu) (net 28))
 (via (at 195.58 57.15) (size 0.8) (drill 0.4) (layers F.Cu B.Cu) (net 28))
 (segment (start 190.5 71.12) (end 190.5 58.42) (width 0.25) (layer B.Cu) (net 28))
 (segment (start 191.77 57.15) (end 195.58 57.15) (width 0.25) (layer B.Cu) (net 28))
 (segment (start 190.5 58.42) (end 191.77 57.15) (width 0.25) (layer B.Cu) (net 28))
 (segment (start 194.31 49.53) (end 194.31 58.024998) (width 0.25) (layer F.Cu) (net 30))
 (segment (start 196.85 46.99) (end 194.31 49.53) (width 0.25) (layer F.Cu) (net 30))
 (segment (start 208.28 46.99) (end 196.85 46.99) (width 0.25) (layer F.Cu) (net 30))
 (segment (start 212.09 43.18) (end 208.28 46.99) (width 0.25) (layer F.Cu) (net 30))
 (segment (start 194.31 58.024998) (end 194.31 62.23) (width 0.25) (layer F.Cu) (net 30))
 (segment (start 218.44 43.18) (end 212.09 43.18) (width 0.25) (layer F.Cu) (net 30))
 (segment (start 219.71 41.91) (end 218.44 43.18) (width 0.25) (layer F.Cu) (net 30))
 (segment (start 220.98 82.55) (end 215.9 82.55) (width 0.25) (layer F.Cu) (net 30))
 (segment (start 215.9 82.55) (end 215.9 82.55) (width 0.25) (layer F.Cu) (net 30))
 (via (at 215.9 82.55) (size 0.8) (drill 0.4) (layers F.Cu B.Cu) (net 30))
 (segment (start 194.31 62.23) (end 194.31 64.77) (width 0.25) (layer F.Cu) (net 30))
 (via (at 194.31 62.23) (size 0.8) (drill 0.4) (layers F.Cu B.Cu) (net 30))
 (segment (start 201.93 81.28) (end 201.93 66.04) (width 0.25) (layer B.Cu) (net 30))
 (segment (start 204.47 83.82) (end 201.93 81.28) (width 0.25) (layer B.Cu) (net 30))
 (segment (start 214.63 83.82) (end 204.47 83.82) (width 0.25) (layer B.Cu) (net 30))
 (segment (start 215.9 82.55) (end 214.63 83.82) (width 0.25) (layer B.Cu) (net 30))
 (segment (start 201.93 66.04) (end 198.12 62.23) (width 0.25) (layer B.Cu) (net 30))
 (segment (start 198.12 62.23) (end 194.31 62.23) (width 0.25) (layer B.Cu) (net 30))
 (segment (start 228.6 39.37) (end 237.49 48.26) (width 0.25) (layer F.Cu) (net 34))
 (segment (start 237.49 48.26) (end 237.79501 48.56501) (width 0.25) (layer F.Cu) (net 34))
 (segment (start 237.79501 73.35499) (end 236.22 74.93) (width 0.25) (layer F.Cu) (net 34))
 (segment (start 240.03 71.12) (end 237.79501 73.35499) (width 0.25) (layer F.Cu) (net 34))
 (segment (start 240.03 50.8) (end 240.03 71.12) (width 0.25) (layer F.Cu) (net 34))
 (segment (start 237.49 48.26) (end 240.03 50.8) (width 0.25) (layer F.Cu) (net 34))
 (segment (start 207.01 41.91) (end 208.28 43.18) (width 0.25) (layer F.Cu) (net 34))
 (segment (start 209.945002 43.18) (end 210.82 42.305002) (width 0.25) (layer F.Cu) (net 34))
 (segment (start 209.55 43.18) (end 209.945002 43.18) (width 0.25) (layer F.Cu) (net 34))
 (segment (start 208.28 43.18) (end 209.55 43.18) (width 0.25) (layer F.Cu) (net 34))
 (segment (start 210.82 42.305002) (end 210.82 41.91) (width 0.25) (layer F.Cu) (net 34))
 (segment (start 210.82 41.91) (end 210.82 40.64) (width 0.25) (layer F.Cu) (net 34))
 (segment (start 210.82 40.64) (end 212.09 39.37) (width 0.25) (layer F.Cu) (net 34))
 (segment (start 212.09 39.37) (end 228.6 39.37) (width 0.25) (layer F.Cu) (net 34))
 (segment (start 220.98 62.23) (end 220.98 59.69) (width 0.25) (layer F.Cu) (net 37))
 (segment (start 217.17 55.88) (end 217.17 49.53) (width 0.25) (layer F.Cu) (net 37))
 (segment (start 220.98 59.69) (end 217.17 55.88) (width 0.25) (layer F.Cu) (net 37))
 (segment (start 220.835001 48.115001) (end 214.63 41.91) (width 0.25) (layer B.Cu) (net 35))
 (segment (start 234.409999 63.355001) (end 220.835001 49.780003) (width 0.25) (layer B.Cu) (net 35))
 (segment (start 236.470003 63.355001) (end 234.409999 63.355001) (width 0.25) (layer B.Cu) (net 35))
 (segment (start 237.345001 64.229999) (end 236.470003 63.355001) (width 0.25) (layer B.Cu) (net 35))
 (segment (start 220.835001 49.780003) (end 220.835001 48.115001) (width 0.25) (layer B.Cu) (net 35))
 (segment (start 237.345001 78.884999) (end 237.345001 64.229999) (width 0.25) (layer B.Cu) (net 35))
 (segment (start 236.22 80.01) (end 237.345001 78.884999) (width 0.25) (layer B.Cu) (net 35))
 (segment (start 216.350009 47.809991) (end 214.63 49.53) (width 0.25) (layer F.Cu) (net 31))
 (segment (start 217.17 46.99) (end 216.350009 47.809991) (width 0.25) (layer F.Cu) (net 31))
 (segment (start 227.33 46.99) (end 217.17 46.99) (width 0.25) (layer F.Cu) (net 31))
 (segment (start 237.49 57.15) (end 227.33 46.99) (width 0.25) (layer F.Cu) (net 31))
 (segment (start 237.49 66.04) (end 237.49 57.15) (width 0.25) (layer F.Cu) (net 31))
 (segment (start 236.22 67.31) (end 237.49 66.04) (width 0.25) (layer F.Cu) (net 31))
 (segment (start 238.76 69.85) (end 236.22 72.39) (width 0.25) (layer F.Cu) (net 33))
 (segment (start 239.57999 69.03001) (end 238.76 69.85) (width 0.25) (layer F.Cu) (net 33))
 (segment (start 239.57999 51.61999) (end 239.57999 69.03001) (width 0.25) (layer F.Cu) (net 33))
 (segment (start 228.6 40.64) (end 239.57999 51.61999) (width 0.25) (layer F.Cu) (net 33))
 (segment (start 219.314998 40.64) (end 228.6 40.64) (width 0.25) (layer F.Cu) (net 33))
 (segment (start 218.044998 41.91) (end 219.314998 40.64) (width 0.25) (layer F.Cu) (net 33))
 (segment (start 217.17 41.91) (end 218.044998 41.91) (width 0.25) (layer F.Cu) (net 33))
 (segment (start 207.01 50.8) (end 207.01 49.53) (width 0.25) (layer F.Cu) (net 36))
 (segment (start 220.98 64.77) (end 207.01 50.8) (width 0.25) (layer F.Cu) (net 36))
 (segment (start 238.30999 67.76001) (end 236.22 69.85) (width 0.25) (layer F.Cu) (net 32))
 (segment (start 238.76 55.88) (end 238.76 67.31) (width 0.25) (layer F.Cu) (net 32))
 (segment (start 238.76 67.31) (end 238.30999 67.76001) (width 0.25) (layer F.Cu) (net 32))
 (segment (start 224.79 41.91) (end 238.76 55.88) (width 0.25) (layer F.Cu) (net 32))
 (segment (start 224.934999 73.515001) (end 236.22 62.23) (width 0.25) (layer F.Cu) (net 9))
 (segment (start 210.675001 73.515001) (end 224.934999 73.515001) (width 0.25) (layer F.Cu) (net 9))
 (segment (start 209.55 72.39) (end 210.675001 73.515001) (width 0.25) (layer F.Cu) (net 9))
 (segment (start 236.22 58.42) (end 227.33 49.53) (width 0.25) (layer F.Cu) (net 9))
 (segment (start 236.22 62.23) (end 236.22 58.42) (width 0.25) (layer F.Cu) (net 9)))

